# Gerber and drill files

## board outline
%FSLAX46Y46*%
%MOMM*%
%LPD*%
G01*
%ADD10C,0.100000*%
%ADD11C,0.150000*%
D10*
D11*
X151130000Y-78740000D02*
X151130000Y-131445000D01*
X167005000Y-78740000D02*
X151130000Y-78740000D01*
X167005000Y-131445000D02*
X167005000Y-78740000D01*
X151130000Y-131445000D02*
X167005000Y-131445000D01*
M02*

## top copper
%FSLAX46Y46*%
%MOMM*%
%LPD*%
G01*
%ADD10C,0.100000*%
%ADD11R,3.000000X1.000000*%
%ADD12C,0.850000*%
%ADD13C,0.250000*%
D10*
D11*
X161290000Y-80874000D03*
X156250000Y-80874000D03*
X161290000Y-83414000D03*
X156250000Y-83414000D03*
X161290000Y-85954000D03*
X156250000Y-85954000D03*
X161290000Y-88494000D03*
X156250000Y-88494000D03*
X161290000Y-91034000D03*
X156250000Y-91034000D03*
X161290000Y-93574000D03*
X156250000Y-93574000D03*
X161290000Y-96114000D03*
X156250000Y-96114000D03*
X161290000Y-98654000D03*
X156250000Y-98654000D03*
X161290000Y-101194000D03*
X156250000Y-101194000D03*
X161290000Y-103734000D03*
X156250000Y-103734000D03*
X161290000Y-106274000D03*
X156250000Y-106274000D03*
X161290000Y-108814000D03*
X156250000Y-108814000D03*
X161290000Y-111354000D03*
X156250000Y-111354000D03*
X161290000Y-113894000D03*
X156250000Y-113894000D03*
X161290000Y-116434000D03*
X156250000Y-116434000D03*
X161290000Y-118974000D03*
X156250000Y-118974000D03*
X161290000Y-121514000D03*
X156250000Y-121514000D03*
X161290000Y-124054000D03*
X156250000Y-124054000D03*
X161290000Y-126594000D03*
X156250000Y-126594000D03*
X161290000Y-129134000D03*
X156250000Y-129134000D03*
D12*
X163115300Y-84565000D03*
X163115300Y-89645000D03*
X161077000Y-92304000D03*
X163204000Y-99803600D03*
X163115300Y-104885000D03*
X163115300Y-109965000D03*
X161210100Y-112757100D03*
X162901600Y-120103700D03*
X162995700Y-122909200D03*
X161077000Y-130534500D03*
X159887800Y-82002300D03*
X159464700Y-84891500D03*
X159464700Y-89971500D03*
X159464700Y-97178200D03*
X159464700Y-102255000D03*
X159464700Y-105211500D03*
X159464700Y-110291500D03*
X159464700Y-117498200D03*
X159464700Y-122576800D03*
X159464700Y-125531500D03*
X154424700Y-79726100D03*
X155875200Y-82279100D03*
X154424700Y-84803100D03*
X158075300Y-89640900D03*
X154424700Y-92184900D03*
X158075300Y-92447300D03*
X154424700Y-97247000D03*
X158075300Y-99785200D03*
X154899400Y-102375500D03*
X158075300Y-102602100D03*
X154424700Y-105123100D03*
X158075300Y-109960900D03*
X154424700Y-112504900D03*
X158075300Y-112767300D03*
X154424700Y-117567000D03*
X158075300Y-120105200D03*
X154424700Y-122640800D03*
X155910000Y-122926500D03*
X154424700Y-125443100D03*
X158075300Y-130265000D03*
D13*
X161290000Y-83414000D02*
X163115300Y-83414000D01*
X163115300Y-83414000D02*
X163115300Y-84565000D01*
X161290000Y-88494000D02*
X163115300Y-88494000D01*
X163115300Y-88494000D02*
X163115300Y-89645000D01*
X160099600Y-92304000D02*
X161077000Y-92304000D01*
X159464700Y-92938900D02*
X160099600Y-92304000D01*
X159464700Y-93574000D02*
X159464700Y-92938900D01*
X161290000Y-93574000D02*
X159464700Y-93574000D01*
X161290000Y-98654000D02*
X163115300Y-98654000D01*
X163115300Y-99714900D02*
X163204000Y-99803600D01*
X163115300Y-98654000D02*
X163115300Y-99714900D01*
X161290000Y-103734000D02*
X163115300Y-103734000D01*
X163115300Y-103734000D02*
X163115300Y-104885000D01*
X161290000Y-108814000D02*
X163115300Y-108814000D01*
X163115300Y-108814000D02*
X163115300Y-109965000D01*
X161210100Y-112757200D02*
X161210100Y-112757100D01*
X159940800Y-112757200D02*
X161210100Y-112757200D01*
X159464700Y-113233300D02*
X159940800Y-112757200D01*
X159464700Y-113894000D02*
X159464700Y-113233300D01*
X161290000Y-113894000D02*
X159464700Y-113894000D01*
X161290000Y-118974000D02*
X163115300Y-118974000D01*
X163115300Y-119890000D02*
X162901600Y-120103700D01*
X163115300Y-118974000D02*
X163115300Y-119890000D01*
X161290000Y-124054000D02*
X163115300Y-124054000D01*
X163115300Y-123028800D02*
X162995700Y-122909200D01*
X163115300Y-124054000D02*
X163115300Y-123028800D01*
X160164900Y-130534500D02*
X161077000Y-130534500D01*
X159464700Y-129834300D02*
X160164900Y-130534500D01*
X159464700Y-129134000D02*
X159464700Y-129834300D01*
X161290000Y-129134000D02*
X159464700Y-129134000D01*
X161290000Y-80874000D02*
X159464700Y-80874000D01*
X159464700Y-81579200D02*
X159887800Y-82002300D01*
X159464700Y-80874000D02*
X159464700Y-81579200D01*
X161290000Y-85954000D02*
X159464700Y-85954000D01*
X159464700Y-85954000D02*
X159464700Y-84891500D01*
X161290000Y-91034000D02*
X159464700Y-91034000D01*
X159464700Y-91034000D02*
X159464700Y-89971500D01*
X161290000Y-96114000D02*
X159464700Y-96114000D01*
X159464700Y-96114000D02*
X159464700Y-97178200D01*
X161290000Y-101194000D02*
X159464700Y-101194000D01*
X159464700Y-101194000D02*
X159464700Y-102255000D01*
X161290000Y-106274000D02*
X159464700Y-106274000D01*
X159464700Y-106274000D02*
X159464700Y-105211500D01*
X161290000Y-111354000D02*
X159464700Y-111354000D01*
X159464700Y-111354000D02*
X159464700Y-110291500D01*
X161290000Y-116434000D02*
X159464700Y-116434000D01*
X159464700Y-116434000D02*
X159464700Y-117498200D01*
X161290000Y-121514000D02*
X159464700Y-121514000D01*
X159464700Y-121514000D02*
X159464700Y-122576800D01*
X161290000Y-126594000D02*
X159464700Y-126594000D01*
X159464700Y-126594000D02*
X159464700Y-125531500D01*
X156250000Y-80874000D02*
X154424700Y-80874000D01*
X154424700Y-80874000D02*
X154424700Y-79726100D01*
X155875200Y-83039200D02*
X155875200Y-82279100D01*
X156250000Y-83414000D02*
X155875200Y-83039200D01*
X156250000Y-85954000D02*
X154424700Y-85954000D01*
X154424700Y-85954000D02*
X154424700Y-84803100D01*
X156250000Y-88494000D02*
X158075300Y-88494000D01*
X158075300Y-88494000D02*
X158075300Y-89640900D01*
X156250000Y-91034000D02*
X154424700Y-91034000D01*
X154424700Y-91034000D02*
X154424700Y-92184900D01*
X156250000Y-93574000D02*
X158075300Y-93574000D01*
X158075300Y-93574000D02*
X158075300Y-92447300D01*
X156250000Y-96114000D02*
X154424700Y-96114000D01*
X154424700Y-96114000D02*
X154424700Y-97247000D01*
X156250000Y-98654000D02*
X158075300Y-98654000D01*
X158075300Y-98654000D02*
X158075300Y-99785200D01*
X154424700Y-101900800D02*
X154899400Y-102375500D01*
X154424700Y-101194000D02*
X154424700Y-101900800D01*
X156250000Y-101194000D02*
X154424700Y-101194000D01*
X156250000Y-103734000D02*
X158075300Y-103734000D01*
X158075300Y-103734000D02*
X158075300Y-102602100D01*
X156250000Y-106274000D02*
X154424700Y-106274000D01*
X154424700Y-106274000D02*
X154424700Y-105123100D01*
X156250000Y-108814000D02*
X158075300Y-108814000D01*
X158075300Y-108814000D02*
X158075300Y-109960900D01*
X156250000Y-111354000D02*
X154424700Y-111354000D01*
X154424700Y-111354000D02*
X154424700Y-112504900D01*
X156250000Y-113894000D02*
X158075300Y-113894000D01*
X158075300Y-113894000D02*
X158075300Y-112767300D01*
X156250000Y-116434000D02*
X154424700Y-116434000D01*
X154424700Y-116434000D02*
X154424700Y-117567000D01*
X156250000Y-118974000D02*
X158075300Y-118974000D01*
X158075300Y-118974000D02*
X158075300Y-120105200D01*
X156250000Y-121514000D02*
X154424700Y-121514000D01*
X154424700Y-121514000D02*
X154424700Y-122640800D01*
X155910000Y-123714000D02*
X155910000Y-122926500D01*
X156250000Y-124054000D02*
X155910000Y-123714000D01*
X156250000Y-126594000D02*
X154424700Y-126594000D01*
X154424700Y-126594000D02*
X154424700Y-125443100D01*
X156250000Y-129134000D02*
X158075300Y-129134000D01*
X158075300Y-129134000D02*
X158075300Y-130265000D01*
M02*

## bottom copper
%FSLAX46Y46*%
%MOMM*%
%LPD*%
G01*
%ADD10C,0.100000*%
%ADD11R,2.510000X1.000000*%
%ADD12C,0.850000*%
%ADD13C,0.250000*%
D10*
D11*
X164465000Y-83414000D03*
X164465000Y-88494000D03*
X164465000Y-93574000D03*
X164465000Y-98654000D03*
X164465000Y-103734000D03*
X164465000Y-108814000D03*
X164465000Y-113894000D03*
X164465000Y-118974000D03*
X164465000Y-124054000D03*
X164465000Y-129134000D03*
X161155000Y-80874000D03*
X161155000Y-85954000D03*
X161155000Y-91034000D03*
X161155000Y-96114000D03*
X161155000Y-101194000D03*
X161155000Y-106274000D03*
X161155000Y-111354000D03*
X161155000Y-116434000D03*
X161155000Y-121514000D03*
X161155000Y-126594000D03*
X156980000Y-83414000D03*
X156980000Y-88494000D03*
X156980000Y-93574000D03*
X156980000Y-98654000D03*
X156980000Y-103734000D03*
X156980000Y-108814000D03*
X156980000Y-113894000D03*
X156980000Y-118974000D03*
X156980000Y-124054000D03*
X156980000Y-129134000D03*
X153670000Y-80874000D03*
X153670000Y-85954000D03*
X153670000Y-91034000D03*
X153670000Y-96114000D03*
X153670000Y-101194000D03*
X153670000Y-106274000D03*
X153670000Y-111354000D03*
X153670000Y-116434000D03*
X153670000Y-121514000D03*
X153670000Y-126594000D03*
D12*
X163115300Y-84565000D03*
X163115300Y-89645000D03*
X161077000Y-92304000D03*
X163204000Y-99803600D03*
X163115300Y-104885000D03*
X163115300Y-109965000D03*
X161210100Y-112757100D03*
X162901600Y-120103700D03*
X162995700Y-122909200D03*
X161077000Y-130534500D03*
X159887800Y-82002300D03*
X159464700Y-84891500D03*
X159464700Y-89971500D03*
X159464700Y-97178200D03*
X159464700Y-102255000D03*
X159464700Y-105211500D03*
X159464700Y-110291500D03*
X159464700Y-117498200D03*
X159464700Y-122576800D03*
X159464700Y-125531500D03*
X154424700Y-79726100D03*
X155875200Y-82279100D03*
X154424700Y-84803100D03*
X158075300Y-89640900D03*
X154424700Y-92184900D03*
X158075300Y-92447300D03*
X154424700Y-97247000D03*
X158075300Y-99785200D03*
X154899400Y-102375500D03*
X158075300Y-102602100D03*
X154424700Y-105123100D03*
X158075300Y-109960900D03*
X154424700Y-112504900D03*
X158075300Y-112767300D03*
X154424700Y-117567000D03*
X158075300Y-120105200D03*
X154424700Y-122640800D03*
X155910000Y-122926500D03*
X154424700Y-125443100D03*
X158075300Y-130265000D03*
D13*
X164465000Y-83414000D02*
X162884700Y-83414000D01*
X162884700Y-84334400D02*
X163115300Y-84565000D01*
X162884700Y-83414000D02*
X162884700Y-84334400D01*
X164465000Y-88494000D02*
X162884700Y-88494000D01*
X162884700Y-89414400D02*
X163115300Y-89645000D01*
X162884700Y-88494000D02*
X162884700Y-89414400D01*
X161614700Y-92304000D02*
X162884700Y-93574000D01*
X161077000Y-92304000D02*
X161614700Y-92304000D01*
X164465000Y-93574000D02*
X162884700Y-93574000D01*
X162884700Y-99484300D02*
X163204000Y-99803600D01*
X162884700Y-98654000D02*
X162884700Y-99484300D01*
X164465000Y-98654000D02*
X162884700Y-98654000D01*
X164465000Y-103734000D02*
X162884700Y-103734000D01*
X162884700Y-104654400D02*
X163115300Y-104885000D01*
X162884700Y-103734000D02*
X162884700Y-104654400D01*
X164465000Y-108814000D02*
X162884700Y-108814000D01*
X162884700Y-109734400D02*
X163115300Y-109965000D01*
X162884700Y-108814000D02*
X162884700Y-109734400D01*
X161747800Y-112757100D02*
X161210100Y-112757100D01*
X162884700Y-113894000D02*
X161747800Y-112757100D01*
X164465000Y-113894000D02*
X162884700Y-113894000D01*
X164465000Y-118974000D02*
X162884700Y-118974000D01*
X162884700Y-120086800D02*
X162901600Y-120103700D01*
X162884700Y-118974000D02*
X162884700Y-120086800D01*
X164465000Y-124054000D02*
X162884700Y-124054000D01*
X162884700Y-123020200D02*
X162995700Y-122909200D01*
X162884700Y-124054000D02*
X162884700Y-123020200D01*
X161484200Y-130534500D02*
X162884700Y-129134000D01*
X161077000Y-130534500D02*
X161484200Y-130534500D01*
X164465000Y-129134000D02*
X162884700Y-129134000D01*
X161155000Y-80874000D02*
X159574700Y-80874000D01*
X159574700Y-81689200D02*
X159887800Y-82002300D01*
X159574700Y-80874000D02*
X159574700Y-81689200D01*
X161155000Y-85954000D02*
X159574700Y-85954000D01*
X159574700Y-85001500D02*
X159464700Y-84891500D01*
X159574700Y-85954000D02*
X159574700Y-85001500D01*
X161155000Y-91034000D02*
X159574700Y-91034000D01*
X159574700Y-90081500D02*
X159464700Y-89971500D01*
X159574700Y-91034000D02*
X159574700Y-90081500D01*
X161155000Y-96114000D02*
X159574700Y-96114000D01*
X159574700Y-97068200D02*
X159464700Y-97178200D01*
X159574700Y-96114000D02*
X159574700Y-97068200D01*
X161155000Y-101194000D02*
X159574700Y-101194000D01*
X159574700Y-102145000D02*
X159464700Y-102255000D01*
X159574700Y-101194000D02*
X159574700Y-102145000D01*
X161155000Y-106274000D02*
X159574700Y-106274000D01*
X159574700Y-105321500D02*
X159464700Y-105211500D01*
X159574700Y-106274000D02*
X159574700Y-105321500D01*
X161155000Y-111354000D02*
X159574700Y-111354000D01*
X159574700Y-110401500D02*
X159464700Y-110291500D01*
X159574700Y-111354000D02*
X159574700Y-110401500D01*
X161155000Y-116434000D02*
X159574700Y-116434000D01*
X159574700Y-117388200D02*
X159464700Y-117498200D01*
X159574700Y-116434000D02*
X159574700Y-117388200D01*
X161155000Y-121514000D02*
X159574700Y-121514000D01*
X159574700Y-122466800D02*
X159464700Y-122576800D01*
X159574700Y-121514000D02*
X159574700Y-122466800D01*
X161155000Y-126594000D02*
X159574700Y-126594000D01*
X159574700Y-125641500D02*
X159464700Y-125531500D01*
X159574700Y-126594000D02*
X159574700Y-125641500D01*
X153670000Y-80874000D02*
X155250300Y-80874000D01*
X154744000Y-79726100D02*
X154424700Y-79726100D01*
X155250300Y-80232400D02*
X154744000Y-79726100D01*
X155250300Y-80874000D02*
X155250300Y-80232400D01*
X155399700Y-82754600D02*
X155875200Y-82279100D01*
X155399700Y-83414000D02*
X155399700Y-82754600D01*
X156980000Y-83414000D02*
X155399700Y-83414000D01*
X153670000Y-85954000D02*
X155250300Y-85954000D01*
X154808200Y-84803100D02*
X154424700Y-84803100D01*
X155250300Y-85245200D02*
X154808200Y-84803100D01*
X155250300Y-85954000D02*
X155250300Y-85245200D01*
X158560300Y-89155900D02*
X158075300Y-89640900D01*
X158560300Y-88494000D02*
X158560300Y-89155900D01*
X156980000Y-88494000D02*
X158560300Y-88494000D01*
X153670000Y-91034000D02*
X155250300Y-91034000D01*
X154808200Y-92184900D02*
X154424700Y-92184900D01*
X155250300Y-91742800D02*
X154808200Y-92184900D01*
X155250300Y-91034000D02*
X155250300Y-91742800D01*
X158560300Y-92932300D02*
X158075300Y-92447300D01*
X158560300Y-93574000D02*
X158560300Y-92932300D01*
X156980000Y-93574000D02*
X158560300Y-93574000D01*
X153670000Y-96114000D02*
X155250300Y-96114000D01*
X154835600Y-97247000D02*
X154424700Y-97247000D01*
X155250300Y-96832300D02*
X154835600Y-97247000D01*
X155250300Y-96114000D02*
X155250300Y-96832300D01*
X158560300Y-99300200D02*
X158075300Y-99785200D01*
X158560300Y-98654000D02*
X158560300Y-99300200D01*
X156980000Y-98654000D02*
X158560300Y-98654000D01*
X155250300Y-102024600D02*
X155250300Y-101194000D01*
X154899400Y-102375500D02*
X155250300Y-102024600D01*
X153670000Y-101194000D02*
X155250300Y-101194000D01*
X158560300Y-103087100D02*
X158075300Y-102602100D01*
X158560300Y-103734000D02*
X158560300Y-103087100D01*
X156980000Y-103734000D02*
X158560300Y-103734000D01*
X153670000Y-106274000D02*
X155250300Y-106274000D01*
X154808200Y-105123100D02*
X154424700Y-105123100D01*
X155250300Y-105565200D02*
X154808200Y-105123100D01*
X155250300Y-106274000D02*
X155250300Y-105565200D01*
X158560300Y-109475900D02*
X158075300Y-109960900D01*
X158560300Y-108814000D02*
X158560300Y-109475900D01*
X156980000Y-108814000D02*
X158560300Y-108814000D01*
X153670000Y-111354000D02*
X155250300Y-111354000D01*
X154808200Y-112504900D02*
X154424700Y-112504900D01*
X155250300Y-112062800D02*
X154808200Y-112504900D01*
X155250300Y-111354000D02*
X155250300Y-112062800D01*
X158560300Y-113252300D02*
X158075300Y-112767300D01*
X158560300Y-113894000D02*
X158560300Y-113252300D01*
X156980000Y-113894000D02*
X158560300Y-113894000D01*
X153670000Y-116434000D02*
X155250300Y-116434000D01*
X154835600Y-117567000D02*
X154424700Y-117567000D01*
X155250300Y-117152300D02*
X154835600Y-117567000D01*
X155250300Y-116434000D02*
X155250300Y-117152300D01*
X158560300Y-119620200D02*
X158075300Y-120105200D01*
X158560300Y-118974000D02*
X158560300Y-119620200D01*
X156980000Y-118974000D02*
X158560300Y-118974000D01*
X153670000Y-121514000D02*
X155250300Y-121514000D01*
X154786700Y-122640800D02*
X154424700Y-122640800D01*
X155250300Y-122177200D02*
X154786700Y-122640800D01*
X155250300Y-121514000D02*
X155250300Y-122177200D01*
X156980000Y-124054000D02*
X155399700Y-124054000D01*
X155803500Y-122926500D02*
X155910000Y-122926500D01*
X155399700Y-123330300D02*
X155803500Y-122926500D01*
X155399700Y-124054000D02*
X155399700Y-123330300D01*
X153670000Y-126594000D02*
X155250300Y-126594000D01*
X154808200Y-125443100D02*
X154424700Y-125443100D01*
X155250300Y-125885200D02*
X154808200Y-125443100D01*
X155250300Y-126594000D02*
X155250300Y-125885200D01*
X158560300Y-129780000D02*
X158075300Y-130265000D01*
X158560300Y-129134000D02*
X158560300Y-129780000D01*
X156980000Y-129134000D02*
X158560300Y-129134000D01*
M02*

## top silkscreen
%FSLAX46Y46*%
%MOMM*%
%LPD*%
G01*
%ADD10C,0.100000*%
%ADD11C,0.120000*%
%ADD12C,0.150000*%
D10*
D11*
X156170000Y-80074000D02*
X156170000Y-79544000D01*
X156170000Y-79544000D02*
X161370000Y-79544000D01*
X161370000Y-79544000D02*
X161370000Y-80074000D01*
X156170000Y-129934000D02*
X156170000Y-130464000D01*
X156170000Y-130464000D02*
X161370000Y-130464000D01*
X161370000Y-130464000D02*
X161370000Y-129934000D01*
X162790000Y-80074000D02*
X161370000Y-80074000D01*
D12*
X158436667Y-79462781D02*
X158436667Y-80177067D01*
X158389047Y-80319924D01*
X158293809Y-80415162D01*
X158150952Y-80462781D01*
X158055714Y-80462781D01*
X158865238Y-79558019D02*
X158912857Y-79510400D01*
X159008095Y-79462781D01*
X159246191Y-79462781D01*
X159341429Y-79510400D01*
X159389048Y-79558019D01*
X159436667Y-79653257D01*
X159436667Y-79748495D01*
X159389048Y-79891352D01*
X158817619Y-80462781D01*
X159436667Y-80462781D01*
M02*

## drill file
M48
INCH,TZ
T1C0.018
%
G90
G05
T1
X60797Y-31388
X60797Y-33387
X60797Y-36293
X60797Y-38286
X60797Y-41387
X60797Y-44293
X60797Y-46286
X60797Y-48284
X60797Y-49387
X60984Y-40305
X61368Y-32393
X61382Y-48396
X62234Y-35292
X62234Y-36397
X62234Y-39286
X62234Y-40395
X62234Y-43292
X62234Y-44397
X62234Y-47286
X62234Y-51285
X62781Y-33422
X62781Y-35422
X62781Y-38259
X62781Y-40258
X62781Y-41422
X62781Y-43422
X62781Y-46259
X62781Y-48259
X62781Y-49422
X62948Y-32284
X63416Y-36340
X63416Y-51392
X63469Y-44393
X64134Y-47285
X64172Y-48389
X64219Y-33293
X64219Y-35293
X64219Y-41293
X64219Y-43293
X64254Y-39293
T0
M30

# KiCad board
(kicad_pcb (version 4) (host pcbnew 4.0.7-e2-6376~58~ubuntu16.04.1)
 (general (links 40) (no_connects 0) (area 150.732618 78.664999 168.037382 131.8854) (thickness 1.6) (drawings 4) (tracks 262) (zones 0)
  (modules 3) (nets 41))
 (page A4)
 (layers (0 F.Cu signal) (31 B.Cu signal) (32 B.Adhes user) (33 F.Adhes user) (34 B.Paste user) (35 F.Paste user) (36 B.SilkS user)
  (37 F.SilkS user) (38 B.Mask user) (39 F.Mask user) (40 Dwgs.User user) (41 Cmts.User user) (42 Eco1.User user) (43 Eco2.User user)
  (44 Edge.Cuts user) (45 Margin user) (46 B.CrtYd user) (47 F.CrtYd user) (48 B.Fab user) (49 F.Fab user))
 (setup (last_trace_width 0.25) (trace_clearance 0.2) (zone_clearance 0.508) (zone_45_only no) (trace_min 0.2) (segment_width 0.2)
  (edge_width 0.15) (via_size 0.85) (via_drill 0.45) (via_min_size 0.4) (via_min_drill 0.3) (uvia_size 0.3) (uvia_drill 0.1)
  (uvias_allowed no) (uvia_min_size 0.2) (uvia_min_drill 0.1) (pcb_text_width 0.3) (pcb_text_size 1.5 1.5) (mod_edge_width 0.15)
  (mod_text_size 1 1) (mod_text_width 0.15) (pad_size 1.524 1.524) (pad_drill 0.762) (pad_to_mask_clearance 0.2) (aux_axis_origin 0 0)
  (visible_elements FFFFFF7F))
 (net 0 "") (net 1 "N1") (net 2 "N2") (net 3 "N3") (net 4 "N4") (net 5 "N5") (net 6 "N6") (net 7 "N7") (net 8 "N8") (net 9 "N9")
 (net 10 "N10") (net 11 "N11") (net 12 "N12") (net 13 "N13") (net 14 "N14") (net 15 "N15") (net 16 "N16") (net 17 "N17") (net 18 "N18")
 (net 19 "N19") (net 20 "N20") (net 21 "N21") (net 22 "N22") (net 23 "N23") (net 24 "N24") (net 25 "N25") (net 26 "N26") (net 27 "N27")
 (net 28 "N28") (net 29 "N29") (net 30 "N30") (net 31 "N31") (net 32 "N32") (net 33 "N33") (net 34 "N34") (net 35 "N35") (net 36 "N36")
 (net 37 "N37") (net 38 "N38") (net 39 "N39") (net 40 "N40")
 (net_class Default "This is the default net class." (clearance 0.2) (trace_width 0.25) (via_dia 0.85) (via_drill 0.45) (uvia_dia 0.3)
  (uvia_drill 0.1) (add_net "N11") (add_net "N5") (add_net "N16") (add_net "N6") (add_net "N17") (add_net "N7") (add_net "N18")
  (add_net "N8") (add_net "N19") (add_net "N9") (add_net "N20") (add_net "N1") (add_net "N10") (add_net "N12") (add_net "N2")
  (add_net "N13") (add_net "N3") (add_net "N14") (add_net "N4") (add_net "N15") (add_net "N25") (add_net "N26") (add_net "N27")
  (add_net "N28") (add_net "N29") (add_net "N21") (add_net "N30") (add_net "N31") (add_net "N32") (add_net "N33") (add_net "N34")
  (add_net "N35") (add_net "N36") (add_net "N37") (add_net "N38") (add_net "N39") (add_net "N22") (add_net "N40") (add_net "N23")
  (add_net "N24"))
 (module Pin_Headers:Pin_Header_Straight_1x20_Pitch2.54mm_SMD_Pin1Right (layer B.Cu) (at 162.81 105.004 180)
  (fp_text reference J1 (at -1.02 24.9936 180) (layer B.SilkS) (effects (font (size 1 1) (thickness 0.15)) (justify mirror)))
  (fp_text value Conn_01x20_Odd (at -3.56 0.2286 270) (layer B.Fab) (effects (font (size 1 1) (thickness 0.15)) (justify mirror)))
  (pad 2 smd rect (at -1.655 21.59 180) (size 2.51 1) (layers B.Cu B.Paste B.Mask) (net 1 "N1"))
  (pad 4 smd rect (at -1.655 16.51 180) (size 2.51 1) (layers B.Cu B.Paste B.Mask) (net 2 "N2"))
  (pad 6 smd rect (at -1.655 11.43 180) (size 2.51 1) (layers B.Cu B.Paste B.Mask) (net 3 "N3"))
  (pad 8 smd rect (at -1.655 6.35 180) (size 2.51 1) (layers B.Cu B.Paste B.Mask) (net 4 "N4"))
  (pad 10 smd rect (at -1.655 1.27 180) (size 2.51 1) (layers B.Cu B.Paste B.Mask) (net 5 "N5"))
  (pad 12 smd rect (at -1.655 -3.81 180) (size 2.51 1) (layers B.Cu B.Paste B.Mask) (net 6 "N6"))
  (pad 14 smd rect (at -1.655 -8.89 180) (size 2.51 1) (layers B.Cu B.Paste B.Mask) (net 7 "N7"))
  (pad 16 smd rect (at -1.655 -13.97 180) (size 2.51 1) (layers B.Cu B.Paste B.Mask) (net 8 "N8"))
  (pad 18 smd rect (at -1.655 -19.05 180) (size 2.51 1) (layers B.Cu B.Paste B.Mask) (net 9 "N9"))
  (pad 20 smd rect (at -1.655 -24.13 180) (size 2.51 1) (layers B.Cu B.Paste B.Mask) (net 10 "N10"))
  (pad 1 smd rect (at 1.655 24.13 180) (size 2.51 1) (layers B.Cu B.Paste B.Mask) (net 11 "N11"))
  (pad 3 smd rect (at 1.655 19.05 180) (size 2.51 1) (layers B.Cu B.Paste B.Mask) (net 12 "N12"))
  (pad 5 smd rect (at 1.655 13.97 180) (size 2.51 1) (layers B.Cu B.Paste B.Mask) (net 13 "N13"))
  (pad 7 smd rect (at 1.655 8.89 180) (size 2.51 1) (layers B.Cu B.Paste B.Mask) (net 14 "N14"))
  (pad 9 smd rect (at 1.655 3.81 180) (size 2.51 1) (layers B.Cu B.Paste B.Mask) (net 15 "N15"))
  (pad 11 smd rect (at 1.655 -1.27 180) (size 2.51 1) (layers B.Cu B.Paste B.Mask) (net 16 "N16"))
  (pad 13 smd rect (at 1.655 -6.35 180) (size 2.51 1) (layers B.Cu B.Paste B.Mask) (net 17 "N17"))
  (pad 15 smd rect (at 1.655 -11.43 180) (size 2.51 1) (layers B.Cu B.Paste B.Mask) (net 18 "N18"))
  (pad 17 smd rect (at 1.655 -16.51 180) (size 2.51 1) (layers B.Cu B.Paste B.Mask) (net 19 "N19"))
  (pad 19 smd rect (at 1.655 -21.59 180) (size 2.51 1) (layers B.Cu B.Paste B.Mask) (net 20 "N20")))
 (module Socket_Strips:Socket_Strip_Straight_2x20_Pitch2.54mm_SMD (layer F.Cu) (at 158.77 105.004)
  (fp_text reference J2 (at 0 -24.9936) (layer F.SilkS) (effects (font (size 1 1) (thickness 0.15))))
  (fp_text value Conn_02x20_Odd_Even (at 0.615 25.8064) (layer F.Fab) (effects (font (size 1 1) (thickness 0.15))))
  (fp_line (start -2.6 -24.93) (end -2.6 -25.46) (layer F.SilkS) (width 0.12))
  (fp_line (start -2.6 -25.46) (end 2.6 -25.46) (layer F.SilkS) (width 0.12))
  (fp_line (start 2.6 -25.46) (end 2.6 -24.93) (layer F.SilkS) (width 0.12))
  (fp_line (start -2.6 24.93) (end -2.6 25.46) (layer F.SilkS) (width 0.12))
  (fp_line (start -2.6 25.46) (end 2.6 25.46) (layer F.SilkS) (width 0.12))
  (fp_line (start 2.6 25.46) (end 2.6 24.93) (layer F.SilkS) (width 0.12))
  (fp_line (start 4.02 -24.93) (end 2.6 -24.93) (layer F.SilkS) (width 0.12))
  (pad 1 smd rect (at 2.52 -24.13) (size 3 1) (layers F.Cu F.Paste F.Mask) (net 11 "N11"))
  (pad 2 smd rect (at -2.52 -24.13) (size 3 1) (layers F.Cu F.Paste F.Mask) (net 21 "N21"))
  (pad 3 smd rect (at 2.52 -21.59) (size 3 1) (layers F.Cu F.Paste F.Mask) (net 1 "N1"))
  (pad 4 smd rect (at -2.52 -21.59) (size 3 1) (layers F.Cu F.Paste F.Mask) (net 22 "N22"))
  (pad 5 smd rect (at 2.52 -19.05) (size 3 1) (layers F.Cu F.Paste F.Mask) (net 12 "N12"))
  (pad 6 smd rect (at -2.52 -19.05) (size 3 1) (layers F.Cu F.Paste F.Mask) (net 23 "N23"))
  (pad 7 smd rect (at 2.52 -16.51) (size 3 1) (layers F.Cu F.Paste F.Mask) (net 2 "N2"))
  (pad 8 smd rect (at -2.52 -16.51) (size 3 1) (layers F.Cu F.Paste F.Mask) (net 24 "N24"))
  (pad 9 smd rect (at 2.52 -13.97) (size 3 1) (layers F.Cu F.Paste F.Mask) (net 13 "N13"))
  (pad 10 smd rect (at -2.52 -13.97) (size 3 1) (layers F.Cu F.Paste F.Mask) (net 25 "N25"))
  (pad 11 smd rect (at 2.52 -11.43) (size 3 1) (layers F.Cu F.Paste F.Mask) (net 3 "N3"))
  (pad 12 smd rect (at -2.52 -11.43) (size 3 1) (layers F.Cu F.Paste F.Mask) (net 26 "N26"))
  (pad 13 smd rect (at 2.52 -8.89) (size 3 1) (layers F.Cu F.Paste F.Mask) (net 14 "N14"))
  (pad 14 smd rect (at -2.52 -8.89) (size 3 1) (layers F.Cu F.Paste F.Mask) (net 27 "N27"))
  (pad 15 smd rect (at 2.52 -6.35) (size 3 1) (layers F.Cu F.Paste F.Mask) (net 4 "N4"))
  (pad 16 smd rect (at -2.52 -6.35) (size 3 1) (layers F.Cu F.Paste F.Mask) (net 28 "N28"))
  (pad 17 smd rect (at 2.52 -3.81) (size 3 1) (layers F.Cu F.Paste F.Mask) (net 15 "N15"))
  (pad 18 smd rect (at -2.52 -3.81) (size 3 1) (layers F.Cu F.Paste F.Mask) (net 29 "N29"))
  (pad 19 smd rect (at 2.52 -1.27) (size 3 1) (layers F.Cu F.Paste F.Mask) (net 5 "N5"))
  (pad 20 smd rect (at -2.52 -1.27) (size 3 1) (layers F.Cu F.Paste F.Mask) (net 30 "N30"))
  (pad 21 smd rect (at 2.52 1.27) (size 3 1) (layers F.Cu F.Paste F.Mask) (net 16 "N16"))
  (pad 22 smd rect (at -2.52 1.27) (size 3 1) (layers F.Cu F.Paste F.Mask) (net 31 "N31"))
  (pad 23 smd rect (at 2.52 3.81) (size 3 1) (layers F.Cu F.Paste F.Mask) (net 6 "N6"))
  (pad 24 smd rect (at -2.52 3.81) (size 3 1) (layers F.Cu F.Paste F.Mask) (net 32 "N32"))
  (pad 25 smd rect (at 2.52 6.35) (size 3 1) (layers F.Cu F.Paste F.Mask) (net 17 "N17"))
  (pad 26 smd rect (at -2.52 6.35) (size 3 1) (layers F.Cu F.Paste F.Mask) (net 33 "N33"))
  (pad 27 smd rect (at 2.52 8.89) (size 3 1) (layers F.Cu F.Paste F.Mask) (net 7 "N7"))
  (pad 28 smd rect (at -2.52 8.89) (size 3 1) (layers F.Cu F.Paste F.Mask) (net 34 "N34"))
  (pad 29 smd rect (at 2.52 11.43) (size 3 1) (layers F.Cu F.Paste F.Mask) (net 18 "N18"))
  (pad 30 smd rect (at -2.52 11.43) (size 3 1) (layers F.Cu F.Paste F.Mask) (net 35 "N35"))
  (pad 31 smd rect (at 2.52 13.97) (size 3 1) (layers F.Cu F.Paste F.Mask) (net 8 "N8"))
  (pad 32 smd rect (at -2.52 13.97) (size 3 1) (layers F.Cu F.Paste F.Mask) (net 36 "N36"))
  (pad 33 smd rect (at 2.52 16.51) (size 3 1) (layers F.Cu F.Paste F.Mask) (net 19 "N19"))
  (pad 34 smd rect (at -2.52 16.51) (size 3 1) (layers F.Cu F.Paste F.Mask) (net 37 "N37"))
  (pad 35 smd rect (at 2.52 19.05) (size 3 1) (layers F.Cu F.Paste F.Mask) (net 9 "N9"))
  (pad 36 smd rect (at -2.52 19.05) (size 3 1) (layers F.Cu F.Paste F.Mask) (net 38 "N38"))
  (pad 37 smd rect (at 2.52 21.59) (size 3 1) (layers F.Cu F.Paste F.Mask) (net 20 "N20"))
  (pad 38 smd rect (at -2.52 21.59) (size 3 1) (layers F.Cu F.Paste F.Mask) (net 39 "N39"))
  (pad 39 smd rect (at 2.52 24.13) (size 3 1) (layers F.Cu F.Paste F.Mask) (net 10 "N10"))
  (pad 40 smd rect (at -2.52 24.13) (size 3 1) (layers F.Cu F.Paste F.Mask) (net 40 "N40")))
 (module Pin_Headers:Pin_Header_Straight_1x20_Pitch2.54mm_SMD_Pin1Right (layer B.Cu) (at 155.325 105.004 180)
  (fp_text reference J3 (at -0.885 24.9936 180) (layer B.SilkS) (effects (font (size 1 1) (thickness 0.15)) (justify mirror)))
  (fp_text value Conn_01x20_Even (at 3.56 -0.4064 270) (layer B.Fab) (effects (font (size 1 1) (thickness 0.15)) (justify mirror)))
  (pad 2 smd rect (at -1.655 21.59 180) (size 2.51 1) (layers B.Cu B.Paste B.Mask) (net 22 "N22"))
  (pad 4 smd rect (at -1.655 16.51 180) (size 2.51 1) (layers B.Cu B.Paste B.Mask) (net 24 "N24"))
  (pad 6 smd rect (at -1.655 11.43 180) (size 2.51 1) (layers B.Cu B.Paste B.Mask) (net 26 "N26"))
  (pad 8 smd rect (at -1.655 6.35 180) (size 2.51 1) (layers B.Cu B.Paste B.Mask) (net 28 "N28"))
  (pad 10 smd rect (at -1.655 1.27 180) (size 2.51 1) (layers B.Cu B.Paste B.Mask) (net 30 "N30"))
  (pad 12 smd rect (at -1.655 -3.81 180) (size 2.51 1) (layers B.Cu B.Paste B.Mask) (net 32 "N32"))
  (pad 14 smd rect (at -1.655 -8.89 180) (size 2.51 1) (layers B.Cu B.Paste B.Mask) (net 34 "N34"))
  (pad 16 smd rect (at -1.655 -13.97 180) (size 2.51 1) (layers B.Cu B.Paste B.Mask) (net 36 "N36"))
  (pad 18 smd rect (at -1.655 -19.05 180) (size 2.51 1) (layers B.Cu B.Paste B.Mask) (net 38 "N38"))
  (pad 20 smd rect (at -1.655 -24.13 180) (size 2.51 1) (layers B.Cu B.Paste B.Mask) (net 40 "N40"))
  (pad 1 smd rect (at 1.655 24.13 180) (size 2.51 1) (layers B.Cu B.Paste B.Mask) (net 21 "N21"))
  (pad 3 smd rect (at 1.655 19.05 180) (size 2.51 1) (layers B.Cu B.Paste B.Mask) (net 23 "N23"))
  (pad 5 smd rect (at 1.655 13.97 180) (size 2.51 1) (layers B.Cu B.Paste B.Mask) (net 25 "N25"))
  (pad 7 smd rect (at 1.655 8.89 180) (size 2.51 1) (layers B.Cu B.Paste B.Mask) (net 27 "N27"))
  (pad 9 smd rect (at 1.655 3.81 180) (size 2.51 1) (layers B.Cu B.Paste B.Mask) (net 29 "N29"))
  (pad 11 smd rect (at 1.655 -1.27 180) (size 2.51 1) (layers B.Cu B.Paste B.Mask) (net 31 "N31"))
  (pad 13 smd rect (at 1.655 -6.35 180) (size 2.51 1) (layers B.Cu B.Paste B.Mask) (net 33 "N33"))
  (pad 15 smd rect (at 1.655 -11.43 180) (size 2.51 1) (layers B.Cu B.Paste B.Mask) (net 35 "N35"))
  (pad 17 smd rect (at 1.655 -16.51 180) (size 2.51 1) (layers B.Cu B.Paste B.Mask) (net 37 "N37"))
  (pad 19 smd rect (at 1.655 -21.59 180) (size 2.51 1) (layers B.Cu B.Paste B.Mask) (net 39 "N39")))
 (gr_line (start 151.13 78.74) (end 151.13 131.445) (layer Edge.Cuts) (width 0.15))
 (gr_line (start 167.005 78.74) (end 151.13 78.74) (layer Edge.Cuts) (width 0.15))
 (gr_line (start 167.005 131.445) (end 167.005 78.74) (layer Edge.Cuts) (width 0.15))
 (gr_line (start 151.13 131.445) (end 167.005 131.445) (layer Edge.Cuts) (width 0.15))
 (via (at 163.1153 84.565) (size 0.85) (layers F.Cu B.Cu) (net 1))
 (segment (start 161.29 83.414) (end 163.1153 83.414) (width 0.25) (layer F.Cu) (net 1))
 (segment (start 164.465 83.414) (end 162.8847 83.414) (width 0.25) (layer B.Cu) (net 1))
 (segment (start 162.8847 84.3344) (end 163.1153 84.565) (width 0.25) (layer B.Cu) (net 1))
 (segment (start 162.8847 83.414) (end 162.8847 84.3344) (width 0.25) (layer B.Cu) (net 1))
 (segment (start 163.1153 83.414) (end 163.1153 84.565) (width 0.25) (layer F.Cu) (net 1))
 (via (at 163.1153 89.645) (size 0.85) (layers F.Cu B.Cu) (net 2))
 (segment (start 161.29 88.494) (end 163.1153 88.494) (width 0.25) (layer F.Cu) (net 2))
 (segment (start 164.465 88.494) (end 162.8847 88.494) (width 0.25) (layer B.Cu) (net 2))
 (segment (start 162.8847 89.4144) (end 163.1153 89.645) (width 0.25) (layer B.Cu) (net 2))
 (segment (start 162.8847 88.494) (end 162.8847 89.4144) (width 0.25) (layer B.Cu) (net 2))
 (segment (start 163.1153 88.494) (end 163.1153 89.645) (width 0.25) (layer F.Cu) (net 2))
 (via (at 161.077 92.304) (size 0.85) (layers F.Cu B.Cu) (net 3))
 (segment (start 160.0996 92.304) (end 161.077 92.304) (width 0.25) (layer F.Cu) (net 3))
 (segment (start 159.4647 92.9389) (end 160.0996 92.304) (width 0.25) (layer F.Cu) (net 3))
 (segment (start 159.4647 93.574) (end 159.4647 92.9389) (width 0.25) (layer F.Cu) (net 3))
 (segment (start 161.6147 92.304) (end 162.8847 93.574) (width 0.25) (layer B.Cu) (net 3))
 (segment (start 161.077 92.304) (end 161.6147 92.304) (width 0.25) (layer B.Cu) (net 3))
 (segment (start 161.29 93.574) (end 159.4647 93.574) (width 0.25) (layer F.Cu) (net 3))
 (segment (start 164.465 93.574) (end 162.8847 93.574) (width 0.25) (layer B.Cu) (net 3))
 (via (at 163.204 99.8036) (size 0.85) (layers F.Cu B.Cu) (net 4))
 (segment (start 161.29 98.654) (end 163.1153 98.654) (width 0.25) (layer F.Cu) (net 4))
 (segment (start 162.8847 99.4843) (end 163.204 99.8036) (width 0.25) (layer B.Cu) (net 4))
 (segment (start 162.8847 98.654) (end 162.8847 99.4843) (width 0.25) (layer B.Cu) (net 4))
 (segment (start 163.1153 99.7149) (end 163.204 99.8036) (width 0.25) (layer F.Cu) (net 4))
 (segment (start 163.1153 98.654) (end 163.1153 99.7149) (width 0.25) (layer F.Cu) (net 4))
 (segment (start 164.465 98.654) (end 162.8847 98.654) (width 0.25) (layer B.Cu) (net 4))
 (via (at 163.1153 104.885) (size 0.85) (layers F.Cu B.Cu) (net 5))
 (segment (start 161.29 103.734) (end 163.1153 103.734) (width 0.25) (layer F.Cu) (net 5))
 (segment (start 164.465 103.734) (end 162.8847 103.734) (width 0.25) (layer B.Cu) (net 5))
 (segment (start 162.8847 104.6544) (end 163.1153 104.885) (width 0.25) (layer B.Cu) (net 5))
 (segment (start 162.8847 103.734) (end 162.8847 104.6544) (width 0.25) (layer B.Cu) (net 5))
 (segment (start 163.1153 103.734) (end 163.1153 104.885) (width 0.25) (layer F.Cu) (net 5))
 (via (at 163.1153 109.965) (size 0.85) (layers F.Cu B.Cu) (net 6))
 (segment (start 161.29 108.814) (end 163.1153 108.814) (width 0.25) (layer F.Cu) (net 6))
 (segment (start 164.465 108.814) (end 162.8847 108.814) (width 0.25) (layer B.Cu) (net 6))
 (segment (start 162.8847 109.7344) (end 163.1153 109.965) (width 0.25) (layer B.Cu) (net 6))
 (segment (start 162.8847 108.814) (end 162.8847 109.7344) (width 0.25) (layer B.Cu) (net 6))
 (segment (start 163.1153 108.814) (end 163.1153 109.965) (width 0.25) (layer F.Cu) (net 6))
 (via (at 161.2101 112.7571) (size 0.85) (layers F.Cu B.Cu) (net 7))
 (segment (start 161.7478 112.7571) (end 161.2101 112.7571) (width 0.25) (layer B.Cu) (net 7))
 (segment (start 162.8847 113.894) (end 161.7478 112.7571) (width 0.25) (layer B.Cu) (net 7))
 (segment (start 161.2101 112.7572) (end 161.2101 112.7571) (width 0.25) (layer F.Cu) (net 7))
 (segment (start 159.9408 112.7572) (end 161.2101 112.7572) (width 0.25) (layer F.Cu) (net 7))
 (segment (start 159.4647 113.2333) (end 159.9408 112.7572) (width 0.25) (layer F.Cu) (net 7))
 (segment (start 159.4647 113.894) (end 159.4647 113.2333) (width 0.25) (layer F.Cu) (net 7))
 (segment (start 161.29 113.894) (end 159.4647 113.894) (width 0.25) (layer F.Cu) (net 7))
 (segment (start 164.465 113.894) (end 162.8847 113.894) (width 0.25) (layer B.Cu) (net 7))
 (via (at 162.9016 120.1037) (size 0.85) (layers F.Cu B.Cu) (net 8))
 (segment (start 161.29 118.974) (end 163.1153 118.974) (width 0.25) (layer F.Cu) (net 8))
 (segment (start 164.465 118.974) (end 162.8847 118.974) (width 0.25) (layer B.Cu) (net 8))
 (segment (start 162.8847 120.0868) (end 162.9016 120.1037) (width 0.25) (layer B.Cu) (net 8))
 (segment (start 162.8847 118.974) (end 162.8847 120.0868) (width 0.25) (layer B.Cu) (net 8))
 (segment (start 163.1153 119.89) (end 162.9016 120.1037) (width 0.25) (layer F.Cu) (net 8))
 (segment (start 163.1153 118.974) (end 163.1153 119.89) (width 0.25) (layer F.Cu) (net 8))
 (via (at 162.9957 122.9092) (size 0.85) (layers F.Cu B.Cu) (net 9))
 (segment (start 161.29 124.054) (end 163.1153 124.054) (width 0.25) (layer F.Cu) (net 9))
 (segment (start 164.465 124.054) (end 162.8847 124.054) (width 0.25) (layer B.Cu) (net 9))
 (segment (start 162.8847 123.0202) (end 162.9957 122.9092) (width 0.25) (layer B.Cu) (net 9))
 (segment (start 162.8847 124.054) (end 162.8847 123.0202) (width 0.25) (layer B.Cu) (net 9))
 (segment (start 163.1153 123.0288) (end 162.9957 122.9092) (width 0.25) (layer F.Cu) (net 9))
 (segment (start 163.1153 124.054) (end 163.1153 123.0288) (width 0.25) (layer F.Cu) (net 9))
 (via (at 161.077 130.5345) (size 0.85) (layers F.Cu B.Cu) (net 10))
 (segment (start 160.1649 130.5345) (end 161.077 130.5345) (width 0.25) (layer F.Cu) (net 10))
 (segment (start 159.4647 129.8343) (end 160.1649 130.5345) (width 0.25) (layer F.Cu) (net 10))
 (segment (start 159.4647 129.134) (end 159.4647 129.8343) (width 0.25) (layer F.Cu) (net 10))
 (segment (start 161.4842 130.5345) (end 162.8847 129.134) (width 0.25) (layer B.Cu) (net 10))
 (segment (start 161.077 130.5345) (end 161.4842 130.5345) (width 0.25) (layer B.Cu) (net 10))
 (segment (start 161.29 129.134) (end 159.4647 129.134) (width 0.25) (layer F.Cu) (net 10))
 (segment (start 164.465 129.134) (end 162.8847 129.134) (width 0.25) (layer B.Cu) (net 10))
 (via (at 159.8878 82.0023) (size 0.85) (layers F.Cu B.Cu) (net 11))
 (segment (start 161.155 80.874) (end 159.5747 80.874) (width 0.25) (layer B.Cu) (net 11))
 (segment (start 161.29 80.874) (end 159.4647 80.874) (width 0.25) (layer F.Cu) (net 11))
 (segment (start 159.5747 81.6892) (end 159.8878 82.0023) (width 0.25) (layer B.Cu) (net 11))
 (segment (start 159.5747 80.874) (end 159.5747 81.6892) (width 0.25) (layer B.Cu) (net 11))
 (segment (start 159.4647 81.5792) (end 159.8878 82.0023) (width 0.25) (layer F.Cu) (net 11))
 (segment (start 159.4647 80.874) (end 159.4647 81.5792) (width 0.25) (layer F.Cu) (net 11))
 (via (at 159.4647 84.8915) (size 0.85) (layers F.Cu B.Cu) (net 12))
 (segment (start 161.29 85.954) (end 159.4647 85.954) (width 0.25) (layer F.Cu) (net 12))
 (segment (start 161.155 85.954) (end 159.5747 85.954) (width 0.25) (layer B.Cu) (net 12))
 (segment (start 159.5747 85.0015) (end 159.4647 84.8915) (width 0.25) (layer B.Cu) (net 12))
 (segment (start 159.5747 85.954) (end 159.5747 85.0015) (width 0.25) (layer B.Cu) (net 12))
 (segment (start 159.4647 85.954) (end 159.4647 84.8915) (width 0.25) (layer F.Cu) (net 12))
 (via (at 159.4647 89.9715) (size 0.85) (layers F.Cu B.Cu) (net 13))
 (segment (start 161.29 91.034) (end 159.4647 91.034) (width 0.25) (layer F.Cu) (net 13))
 (segment (start 161.155 91.034) (end 159.5747 91.034) (width 0.25) (layer B.Cu) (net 13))
 (segment (start 159.5747 90.0815) (end 159.4647 89.9715) (width 0.25) (layer B.Cu) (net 13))
 (segment (start 159.5747 91.034) (end 159.5747 90.0815) (width 0.25) (layer B.Cu) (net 13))
 (segment (start 159.4647 91.034) (end 159.4647 89.9715) (width 0.25) (layer F.Cu) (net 13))
 (via (at 159.4647 97.1782) (size 0.85) (layers F.Cu B.Cu) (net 14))
 (segment (start 161.29 96.114) (end 159.4647 96.114) (width 0.25) (layer F.Cu) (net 14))
 (segment (start 161.155 96.114) (end 159.5747 96.114) (width 0.25) (layer B.Cu) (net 14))
 (segment (start 159.5747 97.0682) (end 159.4647 97.1782) (width 0.25) (layer B.Cu) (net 14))
 (segment (start 159.5747 96.114) (end 159.5747 97.0682) (width 0.25) (layer B.Cu) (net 14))
 (segment (start 159.4647 96.114) (end 159.4647 97.1782) (width 0.25) (layer F.Cu) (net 14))
 (via (at 159.4647 102.255) (size 0.85) (layers F.Cu B.Cu) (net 15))
 (segment (start 161.29 101.194) (end 159.4647 101.194) (width 0.25) (layer F.Cu) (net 15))
 (segment (start 161.155 101.194) (end 159.5747 101.194) (width 0.25) (layer B.Cu) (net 15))
 (segment (start 159.5747 102.145) (end 159.4647 102.255) (width 0.25) (layer B.Cu) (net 15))
 (segment (start 159.5747 101.194) (end 159.5747 102.145) (width 0.25) (layer B.Cu) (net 15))
 (segment (start 159.4647 101.194) (end 159.4647 102.255) (width 0.25) (layer F.Cu) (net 15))
 (via (at 159.4647 105.2115) (size 0.85) (layers F.Cu B.Cu) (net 16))
 (segment (start 161.29 106.274) (end 159.4647 106.274) (width 0.25) (layer F.Cu) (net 16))
 (segment (start 161.155 106.274) (end 159.5747 106.274) (width 0.25) (layer B.Cu) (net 16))
 (segment (start 159.5747 105.3215) (end 159.4647 105.2115) (width 0.25) (layer B.Cu) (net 16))
 (segment (start 159.5747 106.274) (end 159.5747 105.3215) (width 0.25) (layer B.Cu) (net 16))
 (segment (start 159.4647 106.274) (end 159.4647 105.2115) (width 0.25) (layer F.Cu) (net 16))
 (via (at 159.4647 110.2915) (size 0.85) (layers F.Cu B.Cu) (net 17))
 (segment (start 161.29 111.354) (end 159.4647 111.354) (width 0.25) (layer F.Cu) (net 17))
 (segment (start 161.155 111.354) (end 159.5747 111.354) (width 0.25) (layer B.Cu) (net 17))
 (segment (start 159.5747 110.4015) (end 159.4647 110.2915) (width 0.25) (layer B.Cu) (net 17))
 (segment (start 159.5747 111.354) (end 159.5747 110.4015) (width 0.25) (layer B.Cu) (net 17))
 (segment (start 159.4647 111.354) (end 159.4647 110.2915) (width 0.25) (layer F.Cu) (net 17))
 (via (at 159.4647 117.4982) (size 0.85) (layers F.Cu B.Cu) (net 18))
 (segment (start 161.29 116.434) (end 159.4647 116.434) (width 0.25) (layer F.Cu) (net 18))
 (segment (start 161.155 116.434) (end 159.5747 116.434) (width 0.25) (layer B.Cu) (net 18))
 (segment (start 159.5747 117.3882) (end 159.4647 117.4982) (width 0.25) (layer B.Cu) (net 18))
 (segment (start 159.5747 116.434) (end 159.5747 117.3882) (width 0.25) (layer B.Cu) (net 18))
 (segment (start 159.4647 116.434) (end 159.4647 117.4982) (width 0.25) (layer F.Cu) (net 18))
 (via (at 159.4647 122.5768) (size 0.85) (layers F.Cu B.Cu) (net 19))
 (segment (start 161.29 121.514) (end 159.4647 121.514) (width 0.25) (layer F.Cu) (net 19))
 (segment (start 161.155 121.514) (end 159.5747 121.514) (width 0.25) (layer B.Cu) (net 19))
 (segment (start 159.5747 122.4668) (end 159.4647 122.5768) (width 0.25) (layer B.Cu) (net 19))
 (segment (start 159.5747 121.514) (end 159.5747 122.4668) (width 0.25) (layer B.Cu) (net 19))
 (segment (start 159.4647 121.514) (end 159.4647 122.5768) (width 0.25) (layer F.Cu) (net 19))
 (via (at 159.4647 125.5315) (size 0.85) (layers F.Cu B.Cu) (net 20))
 (segment (start 161.29 126.594) (end 159.4647 126.594) (width 0.25) (layer F.Cu) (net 20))
 (segment (start 161.155 126.594) (end 159.5747 126.594) (width 0.25) (layer B.Cu) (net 20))
 (segment (start 159.5747 125.6415) (end 159.4647 125.5315) (width 0.25) (layer B.Cu) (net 20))
 (segment (start 159.5747 126.594) (end 159.5747 125.6415) (width 0.25) (layer B.Cu) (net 20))
 (segment (start 159.4647 126.594) (end 159.4647 125.5315) (width 0.25) (layer F.Cu) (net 20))
 (via (at 154.4247 79.7261) (size 0.85) (layers F.Cu B.Cu) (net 21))
 (segment (start 156.25 80.874) (end 154.4247 80.874) (width 0.25) (layer F.Cu) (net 21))
 (segment (start 153.67 80.874) (end 155.2503 80.874) (width 0.25) (layer B.Cu) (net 21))
 (segment (start 154.744 79.7261) (end 154.4247 79.7261) (width 0.25) (layer B.Cu) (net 21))
 (segment (start 155.2503 80.2324) (end 154.744 79.7261) (width 0.25) (layer B.Cu) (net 21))
 (segment (start 155.2503 80.874) (end 155.2503 80.2324) (width 0.25) (layer B.Cu) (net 21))
 (segment (start 154.4247 80.874) (end 154.4247 79.7261) (width 0.25) (layer F.Cu) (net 21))
 (via (at 155.8752 82.2791) (size 0.85) (layers F.Cu B.Cu) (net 22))
 (segment (start 155.3997 82.7546) (end 155.8752 82.2791) (width 0.25) (layer B.Cu) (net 22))
 (segment (start 155.3997 83.414) (end 155.3997 82.7546) (width 0.25) (layer B.Cu) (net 22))
 (segment (start 155.8752 83.0392) (end 155.8752 82.2791) (width 0.25) (layer F.Cu) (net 22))
 (segment (start 156.25 83.414) (end 155.8752 83.0392) (width 0.25) (layer F.Cu) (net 22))
 (segment (start 156.98 83.414) (end 155.3997 83.414) (width 0.25) (layer B.Cu) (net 22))
 (via (at 154.4247 84.8031) (size 0.85) (layers F.Cu B.Cu) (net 23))
 (segment (start 156.25 85.954) (end 154.4247 85.954) (width 0.25) (layer F.Cu) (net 23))
 (segment (start 153.67 85.954) (end 155.2503 85.954) (width 0.25) (layer B.Cu) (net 23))
 (segment (start 154.8082 84.8031) (end 154.4247 84.8031) (width 0.25) (layer B.Cu) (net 23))
 (segment (start 155.2503 85.2452) (end 154.8082 84.8031) (width 0.25) (layer B.Cu) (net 23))
 (segment (start 155.2503 85.954) (end 155.2503 85.2452) (width 0.25) (layer B.Cu) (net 23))
 (segment (start 154.4247 85.954) (end 154.4247 84.8031) (width 0.25) (layer F.Cu) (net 23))
 (via (at 158.0753 89.6409) (size 0.85) (layers F.Cu B.Cu) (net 24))
 (segment (start 156.25 88.494) (end 158.0753 88.494) (width 0.25) (layer F.Cu) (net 24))
 (segment (start 158.5603 89.1559) (end 158.0753 89.6409) (width 0.25) (layer B.Cu) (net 24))
 (segment (start 158.5603 88.494) (end 158.5603 89.1559) (width 0.25) (layer B.Cu) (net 24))
 (segment (start 158.0753 88.494) (end 158.0753 89.6409) (width 0.25) (layer F.Cu) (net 24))
 (segment (start 156.98 88.494) (end 158.5603 88.494) (width 0.25) (layer B.Cu) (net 24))
 (via (at 154.4247 92.1849) (size 0.85) (layers F.Cu B.Cu) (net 25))
 (segment (start 156.25 91.034) (end 154.4247 91.034) (width 0.25) (layer F.Cu) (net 25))
 (segment (start 153.67 91.034) (end 155.2503 91.034) (width 0.25) (layer B.Cu) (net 25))
 (segment (start 154.8082 92.1849) (end 154.4247 92.1849) (width 0.25) (layer B.Cu) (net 25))
 (segment (start 155.2503 91.7428) (end 154.8082 92.1849) (width 0.25) (layer B.Cu) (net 25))
 (segment (start 155.2503 91.034) (end 155.2503 91.7428) (width 0.25) (layer B.Cu) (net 25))
 (segment (start 154.4247 91.034) (end 154.4247 92.1849) (width 0.25) (layer F.Cu) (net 25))
 (via (at 158.0753 92.4473) (size 0.85) (layers F.Cu B.Cu) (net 26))
 (segment (start 156.25 93.574) (end 158.0753 93.574) (width 0.25) (layer F.Cu) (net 26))
 (segment (start 158.5603 92.9323) (end 158.0753 92.4473) (width 0.25) (layer B.Cu) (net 26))
 (segment (start 158.5603 93.574) (end 158.5603 92.9323) (width 0.25) (layer B.Cu) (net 26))
 (segment (start 158.0753 93.574) (end 158.0753 92.4473) (width 0.25) (layer F.Cu) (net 26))
 (segment (start 156.98 93.574) (end 158.5603 93.574) (width 0.25) (layer B.Cu) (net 26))
 (via (at 154.4247 97.247) (size 0.85) (layers F.Cu B.Cu) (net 27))
 (segment (start 156.25 96.114) (end 154.4247 96.114) (width 0.25) (layer F.Cu) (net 27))
 (segment (start 153.67 96.114) (end 155.2503 96.114) (width 0.25) (layer B.Cu) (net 27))
 (segment (start 154.8356 97.247) (end 154.4247 97.247) (width 0.25) (layer B.Cu) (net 27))
 (segment (start 155.2503 96.8323) (end 154.8356 97.247) (width 0.25) (layer B.Cu) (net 27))
 (segment (start 155.2503 96.114) (end 155.2503 96.8323) (width 0.25) (layer B.Cu) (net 27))
 (segment (start 154.4247 96.114) (end 154.4247 97.247) (width 0.25) (layer F.Cu) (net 27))
 (via (at 158.0753 99.7852) (size 0.85) (layers F.Cu B.Cu) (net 28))
 (segment (start 156.25 98.654) (end 158.0753 98.654) (width 0.25) (layer F.Cu) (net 28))
 (segment (start 158.5603 99.3002) (end 158.0753 99.7852) (width 0.25) (layer B.Cu) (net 28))
 (segment (start 158.5603 98.654) (end 158.5603 99.3002) (width 0.25) (layer B.Cu) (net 28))
 (segment (start 158.0753 98.654) (end 158.0753 99.7852) (width 0.25) (layer F.Cu) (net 28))
 (segment (start 156.98 98.654) (end 158.5603 98.654) (width 0.25) (layer B.Cu) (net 28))
 (via (at 154.8994 102.3755) (size 0.85) (layers F.Cu B.Cu) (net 29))
 (segment (start 154.4247 101.9008) (end 154.8994 102.3755) (width 0.25) (layer F.Cu) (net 29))
 (segment (start 154.4247 101.194) (end 154.4247 101.9008) (width 0.25) (layer F.Cu) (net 29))
 (segment (start 155.2503 102.0246) (end 155.2503 101.194) (width 0.25) (layer B.Cu) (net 29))
 (segment (start 154.8994 102.3755) (end 155.2503 102.0246) (width 0.25) (layer B.Cu) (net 29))
 (segment (start 156.25 101.194) (end 154.4247 101.194) (width 0.25) (layer F.Cu) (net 29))
 (segment (start 153.67 101.194) (end 155.2503 101.194) (width 0.25) (layer B.Cu) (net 29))
 (via (at 158.0753 102.6021) (size 0.85) (layers F.Cu B.Cu) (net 30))
 (segment (start 156.25 103.734) (end 158.0753 103.734) (width 0.25) (layer F.Cu) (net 30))
 (segment (start 158.5603 103.0871) (end 158.0753 102.6021) (width 0.25) (layer B.Cu) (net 30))
 (segment (start 158.5603 103.734) (end 158.5603 103.0871) (width 0.25) (layer B.Cu) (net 30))
 (segment (start 158.0753 103.734) (end 158.0753 102.6021) (width 0.25) (layer F.Cu) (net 30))
 (segment (start 156.98 103.734) (end 158.5603 103.734) (width 0.25) (layer B.Cu) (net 30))
 (via (at 154.4247 105.1231) (size 0.85) (layers F.Cu B.Cu) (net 31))
 (segment (start 156.25 106.274) (end 154.4247 106.274) (width 0.25) (layer F.Cu) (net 31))
 (segment (start 153.67 106.274) (end 155.2503 106.274) (width 0.25) (layer B.Cu) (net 31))
 (segment (start 154.8082 105.1231) (end 154.4247 105.1231) (width 0.25) (layer B.Cu) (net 31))
 (segment (start 155.2503 105.5652) (end 154.8082 105.1231) (width 0.25) (layer B.Cu) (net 31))
 (segment (start 155.2503 106.274) (end 155.2503 105.5652) (width 0.25) (layer B.Cu) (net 31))
 (segment (start 154.4247 106.274) (end 154.4247 105.1231) (width 0.25) (layer F.Cu) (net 31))
 (via (at 158.0753 109.9609) (size 0.85) (layers F.Cu B.Cu) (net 32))
 (segment (start 156.25 108.814) (end 158.0753 108.814) (width 0.25) (layer F.Cu) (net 32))
 (segment (start 158.5603 109.4759) (end 158.0753 109.9609) (width 0.25) (layer B.Cu) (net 32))
 (segment (start 158.5603 108.814) (end 158.5603 109.4759) (width 0.25) (layer B.Cu) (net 32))
 (segment (start 158.0753 108.814) (end 158.0753 109.9609) (width 0.25) (layer F.Cu) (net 32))
 (segment (start 156.98 108.814) (end 158.5603 108.814) (width 0.25) (layer B.Cu) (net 32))
 (via (at 154.4247 112.5049) (size 0.85) (layers F.Cu B.Cu) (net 33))
 (segment (start 156.25 111.354) (end 154.4247 111.354) (width 0.25) (layer F.Cu) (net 33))
 (segment (start 153.67 111.354) (end 155.2503 111.354) (width 0.25) (layer B.Cu) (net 33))
 (segment (start 154.8082 112.5049) (end 154.4247 112.5049) (width 0.25) (layer B.Cu) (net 33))
 (segment (start 155.2503 112.0628) (end 154.8082 112.5049) (width 0.25) (layer B.Cu) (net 33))
 (segment (start 155.2503 111.354) (end 155.2503 112.0628) (width 0.25) (layer B.Cu) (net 33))
 (segment (start 154.4247 111.354) (end 154.4247 112.5049) (width 0.25) (layer F.Cu) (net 33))
 (via (at 158.0753 112.7673) (size 0.85) (layers F.Cu B.Cu) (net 34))
 (segment (start 156.25 113.894) (end 158.0753 113.894) (width 0.25) (layer F.Cu) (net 34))
 (segment (start 158.5603 113.2523) (end 158.0753 112.7673) (width 0.25) (layer B.Cu) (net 34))
 (segment (start 158.5603 113.894) (end 158.5603 113.2523) (width 0.25) (layer B.Cu) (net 34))
 (segment (start 158.0753 113.894) (end 158.0753 112.7673) (width 0.25) (layer F.Cu) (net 34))
 (segment (start 156.98 113.894) (end 158.5603 113.894) (width 0.25) (layer B.Cu) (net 34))
 (via (at 154.4247 117.567) (size 0.85) (layers F.Cu B.Cu) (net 35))
 (segment (start 156.25 116.434) (end 154.4247 116.434) (width 0.25) (layer F.Cu) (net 35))
 (segment (start 153.67 116.434) (end 155.2503 116.434) (width 0.25) (layer B.Cu) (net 35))
 (segment (start 154.8356 117.567) (end 154.4247 117.567) (width 0.25) (layer B.Cu) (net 35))
 (segment (start 155.2503 117.1523) (end 154.8356 117.567) (width 0.25) (layer B.Cu) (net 35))
 (segment (start 155.2503 116.434) (end 155.2503 117.1523) (width 0.25) (layer B.Cu) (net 35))
 (segment (start 154.4247 116.434) (end 154.4247 117.567) (width 0.25) (layer F.Cu) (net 35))
 (via (at 158.0753 120.1052) (size 0.85) (layers F.Cu B.Cu) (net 36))
 (segment (start 156.25 118.974) (end 158.0753 118.974) (width 0.25) (layer F.Cu) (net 36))
 (segment (start 158.5603 119.6202) (end 158.0753 120.1052) (width 0.25) (layer B.Cu) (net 36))
 (segment (start 158.5603 118.974) (end 158.5603 119.6202) (width 0.25) (layer B.Cu) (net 36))
 (segment (start 158.0753 118.974) (end 158.0753 120.1052) (width 0.25) (layer F.Cu) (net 36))
 (segment (start 156.98 118.974) (end 158.5603 118.974) (width 0.25) (layer B.Cu) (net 36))
 (via (at 154.4247 122.6408) (size 0.85) (layers F.Cu B.Cu) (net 37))
 (segment (start 156.25 121.514) (end 154.4247 121.514) (width 0.25) (layer F.Cu) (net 37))
 (segment (start 153.67 121.514) (end 155.2503 121.514) (width 0.25) (layer B.Cu) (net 37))
 (segment (start 154.7867 122.6408) (end 154.4247 122.6408) (width 0.25) (layer B.Cu) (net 37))
 (segment (start 155.2503 122.1772) (end 154.7867 122.6408) (width 0.25) (layer B.Cu) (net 37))
 (segment (start 155.2503 121.514) (end 155.2503 122.1772) (width 0.25) (layer B.Cu) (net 37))
 (segment (start 154.4247 121.514) (end 154.4247 122.6408) (width 0.25) (layer F.Cu) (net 37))
 (via (at 155.91 122.9265) (size 0.85) (layers F.Cu B.Cu) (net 38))
 (segment (start 156.98 124.054) (end 155.3997 124.054) (width 0.25) (layer B.Cu) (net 38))
 (segment (start 155.8035 122.9265) (end 155.91 122.9265) (width 0.25) (layer B.Cu) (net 38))
 (segment (start 155.3997 123.3303) (end 155.8035 122.9265) (width 0.25) (layer B.Cu) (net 38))
 (segment (start 155.3997 124.054) (end 155.3997 123.3303) (width 0.25) (layer B.Cu) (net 38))
 (segment (start 155.91 123.714) (end 155.91 122.9265) (width 0.25) (layer F.Cu) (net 38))
 (segment (start 156.25 124.054) (end 155.91 123.714) (width 0.25) (layer F.Cu) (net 38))
 (via (at 154.4247 125.4431) (size 0.85) (layers F.Cu B.Cu) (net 39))
 (segment (start 156.25 126.594) (end 154.4247 126.594) (width 0.25) (layer F.Cu) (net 39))
 (segment (start 153.67 126.594) (end 155.2503 126.594) (width 0.25) (layer B.Cu) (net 39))
 (segment (start 154.8082 125.4431) (end 154.4247 125.4431) (width 0.25) (layer B.Cu) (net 39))
 (segment (start 155.2503 125.8852) (end 154.8082 125.4431) (width 0.25) (layer B.Cu) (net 39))
 (segment (start 155.2503 126.594) (end 155.2503 125.8852) (width 0.25) (layer B.Cu) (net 39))
 (segment (start 154.4247 126.594) (end 154.4247 125.4431) (width 0.25) (layer F.Cu) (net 39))
 (via (at 158.0753 130.265) (size 0.85) (layers F.Cu B.Cu) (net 40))
 (segment (start 156.25 129.134) (end 158.0753 129.134) (width 0.25) (layer F.Cu) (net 40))
 (segment (start 158.5603 129.78) (end 158.0753 130.265) (width 0.25) (layer B.Cu) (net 40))
 (segment (start 158.5603 129.134) (end 158.5603 129.78) (width 0.25) (layer B.Cu) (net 40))
 (segment (start 158.0753 129.134) (end 158.0753 130.265) (width 0.25) (layer F.Cu) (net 40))
 (segment (start 156.98 129.134) (end 158.5603 129.134) (width 0.25) (layer B.Cu) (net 40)))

